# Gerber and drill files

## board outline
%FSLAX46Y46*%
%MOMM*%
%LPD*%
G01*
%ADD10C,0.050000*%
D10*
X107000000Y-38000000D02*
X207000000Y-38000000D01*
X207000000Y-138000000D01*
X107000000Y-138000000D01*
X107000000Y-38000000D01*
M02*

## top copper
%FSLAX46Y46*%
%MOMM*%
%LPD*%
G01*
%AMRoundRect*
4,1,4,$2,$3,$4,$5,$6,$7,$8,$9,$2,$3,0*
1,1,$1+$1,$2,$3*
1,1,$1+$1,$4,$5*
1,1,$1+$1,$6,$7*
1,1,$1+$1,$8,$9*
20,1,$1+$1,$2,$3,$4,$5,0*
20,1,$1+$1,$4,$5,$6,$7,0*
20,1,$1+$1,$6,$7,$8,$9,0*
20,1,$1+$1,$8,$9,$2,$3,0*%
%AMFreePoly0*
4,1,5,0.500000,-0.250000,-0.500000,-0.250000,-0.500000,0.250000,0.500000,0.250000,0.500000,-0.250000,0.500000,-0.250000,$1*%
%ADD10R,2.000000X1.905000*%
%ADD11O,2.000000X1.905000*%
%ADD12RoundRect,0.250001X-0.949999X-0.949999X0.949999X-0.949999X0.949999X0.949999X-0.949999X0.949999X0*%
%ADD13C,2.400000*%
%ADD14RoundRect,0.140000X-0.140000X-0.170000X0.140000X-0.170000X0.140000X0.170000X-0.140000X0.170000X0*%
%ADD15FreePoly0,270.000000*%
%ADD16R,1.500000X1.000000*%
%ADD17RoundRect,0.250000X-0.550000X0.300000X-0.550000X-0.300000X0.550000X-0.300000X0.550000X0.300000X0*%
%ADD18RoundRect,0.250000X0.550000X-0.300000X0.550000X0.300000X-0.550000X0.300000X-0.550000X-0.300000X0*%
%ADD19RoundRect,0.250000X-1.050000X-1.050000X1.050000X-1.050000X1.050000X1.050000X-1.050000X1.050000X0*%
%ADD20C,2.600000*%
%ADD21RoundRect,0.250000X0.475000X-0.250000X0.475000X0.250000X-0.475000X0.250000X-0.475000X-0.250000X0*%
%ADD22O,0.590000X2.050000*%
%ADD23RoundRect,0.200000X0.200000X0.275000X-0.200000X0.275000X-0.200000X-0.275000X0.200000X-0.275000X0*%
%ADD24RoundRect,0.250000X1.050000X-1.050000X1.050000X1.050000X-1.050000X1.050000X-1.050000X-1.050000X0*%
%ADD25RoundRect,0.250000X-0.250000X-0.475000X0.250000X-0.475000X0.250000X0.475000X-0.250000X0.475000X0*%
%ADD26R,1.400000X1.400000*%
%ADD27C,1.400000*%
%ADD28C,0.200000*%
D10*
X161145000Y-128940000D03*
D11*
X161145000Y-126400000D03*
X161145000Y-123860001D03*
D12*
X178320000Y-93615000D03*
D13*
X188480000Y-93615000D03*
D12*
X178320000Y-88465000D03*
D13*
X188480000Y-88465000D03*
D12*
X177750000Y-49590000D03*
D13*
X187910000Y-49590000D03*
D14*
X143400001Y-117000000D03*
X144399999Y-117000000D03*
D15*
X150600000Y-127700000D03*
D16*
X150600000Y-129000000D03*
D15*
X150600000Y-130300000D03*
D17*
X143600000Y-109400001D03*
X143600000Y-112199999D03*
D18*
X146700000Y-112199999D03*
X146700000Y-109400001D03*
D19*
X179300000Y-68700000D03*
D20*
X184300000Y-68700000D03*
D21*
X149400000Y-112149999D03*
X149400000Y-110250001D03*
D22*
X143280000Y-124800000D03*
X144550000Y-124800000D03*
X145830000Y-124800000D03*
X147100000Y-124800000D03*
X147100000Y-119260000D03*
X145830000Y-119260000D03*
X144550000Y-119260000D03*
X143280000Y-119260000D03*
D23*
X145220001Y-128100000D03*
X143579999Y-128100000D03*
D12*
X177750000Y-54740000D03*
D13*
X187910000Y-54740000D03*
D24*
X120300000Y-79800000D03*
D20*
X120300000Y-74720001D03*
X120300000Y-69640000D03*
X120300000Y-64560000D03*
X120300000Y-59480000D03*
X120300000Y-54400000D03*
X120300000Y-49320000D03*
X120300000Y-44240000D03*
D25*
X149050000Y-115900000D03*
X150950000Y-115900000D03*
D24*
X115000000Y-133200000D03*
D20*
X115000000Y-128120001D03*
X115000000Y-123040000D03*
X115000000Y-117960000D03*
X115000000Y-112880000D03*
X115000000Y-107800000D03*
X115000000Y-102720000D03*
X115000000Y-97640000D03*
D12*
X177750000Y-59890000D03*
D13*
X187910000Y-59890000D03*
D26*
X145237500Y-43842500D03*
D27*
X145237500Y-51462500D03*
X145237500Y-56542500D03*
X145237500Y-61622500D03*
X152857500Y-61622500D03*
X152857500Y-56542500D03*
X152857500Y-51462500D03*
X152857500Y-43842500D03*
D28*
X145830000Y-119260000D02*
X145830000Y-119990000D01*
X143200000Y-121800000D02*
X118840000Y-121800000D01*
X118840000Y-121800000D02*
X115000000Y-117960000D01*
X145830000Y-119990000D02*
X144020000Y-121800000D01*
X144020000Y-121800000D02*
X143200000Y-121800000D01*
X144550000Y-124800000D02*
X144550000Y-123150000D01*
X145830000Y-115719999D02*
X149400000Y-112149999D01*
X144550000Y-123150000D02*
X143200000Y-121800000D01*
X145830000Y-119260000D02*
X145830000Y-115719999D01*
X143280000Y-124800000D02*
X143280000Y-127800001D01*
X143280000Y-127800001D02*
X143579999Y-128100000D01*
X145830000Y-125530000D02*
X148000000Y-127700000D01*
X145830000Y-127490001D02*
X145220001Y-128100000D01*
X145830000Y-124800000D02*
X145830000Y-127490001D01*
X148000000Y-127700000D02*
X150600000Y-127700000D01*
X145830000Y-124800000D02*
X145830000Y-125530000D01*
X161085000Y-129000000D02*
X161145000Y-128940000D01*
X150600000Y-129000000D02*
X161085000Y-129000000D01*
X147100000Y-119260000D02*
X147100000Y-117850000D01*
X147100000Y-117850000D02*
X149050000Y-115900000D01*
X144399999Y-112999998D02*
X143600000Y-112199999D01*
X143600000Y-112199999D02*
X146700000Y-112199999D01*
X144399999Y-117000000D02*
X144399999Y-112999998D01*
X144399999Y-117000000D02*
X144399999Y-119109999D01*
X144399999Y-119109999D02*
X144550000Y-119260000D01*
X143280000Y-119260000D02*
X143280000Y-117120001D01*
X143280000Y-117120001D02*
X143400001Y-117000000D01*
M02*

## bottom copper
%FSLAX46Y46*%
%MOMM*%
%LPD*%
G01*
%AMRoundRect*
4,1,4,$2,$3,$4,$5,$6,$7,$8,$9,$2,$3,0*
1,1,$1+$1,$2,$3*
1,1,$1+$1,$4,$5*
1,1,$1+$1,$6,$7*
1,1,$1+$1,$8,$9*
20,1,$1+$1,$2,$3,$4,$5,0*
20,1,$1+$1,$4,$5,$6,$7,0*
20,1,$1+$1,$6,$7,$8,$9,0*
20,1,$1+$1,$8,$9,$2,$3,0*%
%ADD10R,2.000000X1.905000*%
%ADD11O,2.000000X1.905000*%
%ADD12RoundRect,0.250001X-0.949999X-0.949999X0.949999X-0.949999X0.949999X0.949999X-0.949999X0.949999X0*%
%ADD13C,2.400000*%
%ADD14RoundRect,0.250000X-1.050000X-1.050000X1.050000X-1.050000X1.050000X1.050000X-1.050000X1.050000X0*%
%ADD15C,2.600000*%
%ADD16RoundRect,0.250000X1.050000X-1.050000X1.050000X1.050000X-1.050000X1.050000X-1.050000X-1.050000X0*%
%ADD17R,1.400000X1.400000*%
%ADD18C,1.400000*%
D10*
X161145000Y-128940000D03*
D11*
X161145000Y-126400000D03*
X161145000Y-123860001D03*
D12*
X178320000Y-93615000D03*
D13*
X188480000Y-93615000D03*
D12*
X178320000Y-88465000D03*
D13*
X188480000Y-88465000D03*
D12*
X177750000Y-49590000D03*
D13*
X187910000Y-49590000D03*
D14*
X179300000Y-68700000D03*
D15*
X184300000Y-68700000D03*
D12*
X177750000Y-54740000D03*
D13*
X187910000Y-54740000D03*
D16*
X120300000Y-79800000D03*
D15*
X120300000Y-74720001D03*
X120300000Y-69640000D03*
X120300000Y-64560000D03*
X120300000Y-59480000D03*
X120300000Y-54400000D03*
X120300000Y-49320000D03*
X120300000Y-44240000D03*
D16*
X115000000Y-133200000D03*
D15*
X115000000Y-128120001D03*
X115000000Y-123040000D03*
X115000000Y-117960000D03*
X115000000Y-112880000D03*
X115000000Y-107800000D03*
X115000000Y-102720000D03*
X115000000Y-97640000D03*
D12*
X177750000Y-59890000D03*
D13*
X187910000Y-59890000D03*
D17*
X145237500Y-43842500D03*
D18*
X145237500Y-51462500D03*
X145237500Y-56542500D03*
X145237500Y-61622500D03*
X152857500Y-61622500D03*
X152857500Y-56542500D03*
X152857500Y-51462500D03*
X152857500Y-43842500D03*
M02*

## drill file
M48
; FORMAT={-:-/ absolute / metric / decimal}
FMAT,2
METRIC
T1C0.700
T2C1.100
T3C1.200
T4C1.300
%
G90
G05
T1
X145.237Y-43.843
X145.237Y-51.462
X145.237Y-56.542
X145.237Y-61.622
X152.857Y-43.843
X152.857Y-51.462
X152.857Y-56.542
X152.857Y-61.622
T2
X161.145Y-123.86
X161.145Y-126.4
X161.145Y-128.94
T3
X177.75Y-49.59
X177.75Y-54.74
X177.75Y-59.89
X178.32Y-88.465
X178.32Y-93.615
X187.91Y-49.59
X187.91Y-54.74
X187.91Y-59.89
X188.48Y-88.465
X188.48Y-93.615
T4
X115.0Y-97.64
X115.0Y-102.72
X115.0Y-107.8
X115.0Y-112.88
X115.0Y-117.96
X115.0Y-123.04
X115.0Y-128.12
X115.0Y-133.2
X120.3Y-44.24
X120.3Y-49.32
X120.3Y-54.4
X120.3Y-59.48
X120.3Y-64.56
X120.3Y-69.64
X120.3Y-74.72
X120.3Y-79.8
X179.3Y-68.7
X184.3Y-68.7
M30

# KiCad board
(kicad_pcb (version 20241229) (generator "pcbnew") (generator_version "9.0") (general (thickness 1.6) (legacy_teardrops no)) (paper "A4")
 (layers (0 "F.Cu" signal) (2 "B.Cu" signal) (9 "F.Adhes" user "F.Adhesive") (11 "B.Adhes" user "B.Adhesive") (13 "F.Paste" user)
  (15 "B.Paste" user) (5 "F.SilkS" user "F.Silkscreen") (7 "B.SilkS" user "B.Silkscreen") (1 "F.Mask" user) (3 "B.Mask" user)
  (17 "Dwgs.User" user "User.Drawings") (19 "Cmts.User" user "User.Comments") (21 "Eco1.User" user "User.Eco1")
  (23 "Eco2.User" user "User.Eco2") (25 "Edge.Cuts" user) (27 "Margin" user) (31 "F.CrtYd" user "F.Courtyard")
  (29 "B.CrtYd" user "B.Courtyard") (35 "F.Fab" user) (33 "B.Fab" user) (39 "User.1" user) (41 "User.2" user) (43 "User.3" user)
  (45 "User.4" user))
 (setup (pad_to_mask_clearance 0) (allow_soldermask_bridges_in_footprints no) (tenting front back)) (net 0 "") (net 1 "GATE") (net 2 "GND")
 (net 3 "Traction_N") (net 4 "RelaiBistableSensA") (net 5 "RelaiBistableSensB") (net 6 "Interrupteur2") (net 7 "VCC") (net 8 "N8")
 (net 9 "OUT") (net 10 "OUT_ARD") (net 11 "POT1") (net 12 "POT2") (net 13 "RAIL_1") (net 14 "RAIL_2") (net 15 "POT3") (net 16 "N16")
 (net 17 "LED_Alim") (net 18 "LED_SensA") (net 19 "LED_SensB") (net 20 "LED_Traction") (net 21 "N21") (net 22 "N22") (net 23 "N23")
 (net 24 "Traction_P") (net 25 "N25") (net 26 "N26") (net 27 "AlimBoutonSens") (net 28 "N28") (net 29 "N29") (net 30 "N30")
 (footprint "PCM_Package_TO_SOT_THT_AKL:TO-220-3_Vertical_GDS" (layer "F.Cu") (at 161.145 128.94 90)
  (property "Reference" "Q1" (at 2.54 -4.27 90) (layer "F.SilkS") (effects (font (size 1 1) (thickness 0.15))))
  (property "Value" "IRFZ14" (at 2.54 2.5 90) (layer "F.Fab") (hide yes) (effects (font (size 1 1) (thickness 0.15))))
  (pad "1" thru_hole rect (at 0 0 90) (size 1.905 2) (drill 1.1) (layers "*.Cu" "*.Mask") (remove_unused_layers no) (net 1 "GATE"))
  (pad "2" thru_hole oval (at 2.54 0 90) (size 1.905 2) (drill 1.1) (layers "*.Cu" "*.Mask") (remove_unused_layers no) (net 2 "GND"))
  (pad "3" thru_hole oval (at 5.079999 0 90) (size 1.905 2) (drill 1.1) (layers "*.Cu" "*.Mask") (remove_unused_layers no)
   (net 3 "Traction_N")))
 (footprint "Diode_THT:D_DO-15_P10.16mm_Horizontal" (layer "F.Cu") (at 178.32 93.615)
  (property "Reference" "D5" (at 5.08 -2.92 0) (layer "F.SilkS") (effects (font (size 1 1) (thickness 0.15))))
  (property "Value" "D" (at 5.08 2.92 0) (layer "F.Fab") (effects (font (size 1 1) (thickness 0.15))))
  (pad "1" thru_hole roundrect (at 0 0) (size 2.4 2.4) (drill 1.2) (layers "*.Cu" "*.Mask") (remove_unused_layers no)
   (roundrect_rratio 0.104167) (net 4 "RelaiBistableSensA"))
  (pad "2" thru_hole circle (at 10.16 0) (size 2.4 2.4) (drill 1.2) (layers "*.Cu" "*.Mask") (remove_unused_layers no) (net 2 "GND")))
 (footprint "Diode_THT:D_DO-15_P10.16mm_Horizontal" (layer "F.Cu") (at 178.32 88.465)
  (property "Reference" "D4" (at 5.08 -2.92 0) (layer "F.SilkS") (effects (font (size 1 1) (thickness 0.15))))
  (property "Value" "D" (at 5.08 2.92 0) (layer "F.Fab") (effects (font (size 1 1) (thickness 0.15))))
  (pad "1" thru_hole roundrect (at 0 0) (size 2.4 2.4) (drill 1.2) (layers "*.Cu" "*.Mask") (remove_unused_layers no)
   (roundrect_rratio 0.104167) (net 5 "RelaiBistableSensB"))
  (pad "2" thru_hole circle (at 10.16 0) (size 2.4 2.4) (drill 1.2) (layers "*.Cu" "*.Mask") (remove_unused_layers no) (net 2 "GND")))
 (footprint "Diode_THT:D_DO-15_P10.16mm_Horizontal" (layer "F.Cu") (at 177.75 49.59)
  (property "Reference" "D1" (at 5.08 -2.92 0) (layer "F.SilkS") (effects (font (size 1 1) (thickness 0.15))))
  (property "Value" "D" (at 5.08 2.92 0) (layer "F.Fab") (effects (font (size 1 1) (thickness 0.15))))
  (pad "1" thru_hole roundrect (at 0 0) (size 2.4 2.4) (drill 1.2) (layers "*.Cu" "*.Mask") (remove_unused_layers no)
   (roundrect_rratio 0.104167) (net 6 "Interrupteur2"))
  (pad "2" thru_hole circle (at 10.16 0) (size 2.4 2.4) (drill 1.2) (layers "*.Cu" "*.Mask") (remove_unused_layers no) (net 2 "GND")))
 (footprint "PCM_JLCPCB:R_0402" (layer "F.Cu") (at 143.9 117)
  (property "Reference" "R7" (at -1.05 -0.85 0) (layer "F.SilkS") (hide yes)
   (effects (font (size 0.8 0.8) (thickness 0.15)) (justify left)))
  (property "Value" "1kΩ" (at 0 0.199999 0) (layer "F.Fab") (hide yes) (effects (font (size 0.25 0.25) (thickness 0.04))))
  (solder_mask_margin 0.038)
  (pad "1" smd roundrect (at -0.499999 0) (size 0.56 0.62) (layers "F.Cu" "F.Mask" "F.Paste") (roundrect_rratio 0.25) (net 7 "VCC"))
  (pad "2" smd roundrect (at 0.499999 0) (size 0.56 0.62) (layers "F.Cu" "F.Mask" "F.Paste") (roundrect_rratio 0.25) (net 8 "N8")))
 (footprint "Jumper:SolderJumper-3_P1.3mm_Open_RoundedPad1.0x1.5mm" (layer "F.Cu") (at 150.6 129 -90)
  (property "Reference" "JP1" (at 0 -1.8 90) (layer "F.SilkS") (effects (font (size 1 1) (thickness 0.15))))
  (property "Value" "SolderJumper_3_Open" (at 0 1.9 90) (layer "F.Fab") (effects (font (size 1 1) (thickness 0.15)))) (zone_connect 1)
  (pad "1" smd custom (at -1.3 0 270) (size 1 0.5) (layers "F.Cu" "F.Mask") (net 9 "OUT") (zone_connect 2) (thermal_bridge_angle 45)
   (options (clearance outline) (anchor rect)) (primitives))
  (pad "2" smd rect (at 0 0 270) (size 1 1.5) (layers "F.Cu" "F.Mask") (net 1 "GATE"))
  (pad "3" smd custom (at 1.3 0 270) (size 1 0.5) (layers "F.Cu" "F.Mask") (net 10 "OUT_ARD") (zone_connect 2) (thermal_bridge_angle 45)
   (options (clearance outline) (anchor rect)) (primitives)))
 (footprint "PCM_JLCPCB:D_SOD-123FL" (layer "F.Cu") (at 143.6 110.8 -90)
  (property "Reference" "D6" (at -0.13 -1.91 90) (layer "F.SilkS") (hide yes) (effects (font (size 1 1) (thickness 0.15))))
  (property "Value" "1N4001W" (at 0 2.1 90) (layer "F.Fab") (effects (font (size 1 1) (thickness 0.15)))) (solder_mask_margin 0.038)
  (pad "1" smd roundrect (at -1.399999 0 270) (size 1.1 1.6) (layers "F.Cu" "F.Mask" "F.Paste") (roundrect_rratio 0.2272727273)
   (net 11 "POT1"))
  (pad "2" smd roundrect (at 1.399999 0 270) (size 1.1 1.6) (layers "F.Cu" "F.Mask" "F.Paste") (roundrect_rratio 0.2272727273) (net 8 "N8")))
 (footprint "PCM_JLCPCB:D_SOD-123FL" (layer "F.Cu") (at 146.7 110.8 90)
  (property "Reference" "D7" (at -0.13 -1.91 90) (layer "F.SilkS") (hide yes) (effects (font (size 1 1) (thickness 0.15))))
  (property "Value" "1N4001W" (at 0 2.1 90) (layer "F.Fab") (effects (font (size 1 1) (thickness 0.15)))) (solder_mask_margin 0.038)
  (pad "1" smd roundrect (at -1.399999 0 90) (size 1.1 1.6) (layers "F.Cu" "F.Mask" "F.Paste") (roundrect_rratio 0.2272727273) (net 8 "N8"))
  (pad "2" smd roundrect (at 1.399999 0 90) (size 1.1 1.6) (layers "F.Cu" "F.Mask" "F.Paste") (roundrect_rratio 0.2272727273)
   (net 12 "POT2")))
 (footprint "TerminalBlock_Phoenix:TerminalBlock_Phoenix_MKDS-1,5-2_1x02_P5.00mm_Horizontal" (layer "F.Cu") (at 179.3 68.7)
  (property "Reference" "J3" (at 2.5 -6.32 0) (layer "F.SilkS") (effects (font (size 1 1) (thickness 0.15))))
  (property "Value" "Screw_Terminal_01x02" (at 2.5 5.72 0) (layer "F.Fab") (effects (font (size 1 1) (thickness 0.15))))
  (pad "1" thru_hole roundrect (at 0 0) (size 2.6 2.6) (drill 1.3) (layers "*.Cu" "*.Mask") (remove_unused_layers no)
   (roundrect_rratio 0.096154) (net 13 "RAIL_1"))
  (pad "2" thru_hole circle (at 5 0) (size 2.6 2.6) (drill 1.3) (layers "*.Cu" "*.Mask") (remove_unused_layers no) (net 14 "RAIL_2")))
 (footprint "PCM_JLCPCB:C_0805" (layer "F.Cu") (at 149.4 111.2 90)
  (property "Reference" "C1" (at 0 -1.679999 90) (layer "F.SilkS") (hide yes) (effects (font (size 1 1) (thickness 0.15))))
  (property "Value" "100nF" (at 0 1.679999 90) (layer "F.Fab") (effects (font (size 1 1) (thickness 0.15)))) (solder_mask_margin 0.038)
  (pad "1" smd roundrect (at -0.949999 0 90) (size 1 1.45) (layers "F.Cu" "F.Mask" "F.Paste") (roundrect_rratio 0.25) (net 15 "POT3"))
  (pad "2" smd roundrect (at 0.949999 0 90) (size 1 1.45) (layers "F.Cu" "F.Mask" "F.Paste") (roundrect_rratio 0.25) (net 2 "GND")))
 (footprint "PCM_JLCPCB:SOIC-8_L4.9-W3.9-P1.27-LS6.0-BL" (layer "F.Cu") (at 145.19 122.03)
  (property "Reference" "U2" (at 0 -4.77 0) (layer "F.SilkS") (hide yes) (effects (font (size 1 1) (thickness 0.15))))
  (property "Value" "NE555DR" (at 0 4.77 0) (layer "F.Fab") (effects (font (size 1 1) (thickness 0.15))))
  (pad "1" smd oval (at -1.91 2.77) (size 0.59 2.05) (layers "F.Cu" "F.Mask" "F.Paste") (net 2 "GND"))
  (pad "2" smd oval (at -0.64 2.77) (size 0.59 2.05) (layers "F.Cu" "F.Mask" "F.Paste") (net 15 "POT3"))
  (pad "3" smd oval (at 0.64 2.77) (size 0.59 2.05) (layers "F.Cu" "F.Mask" "F.Paste") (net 9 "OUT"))
  (pad "4" smd oval (at 1.91 2.77) (size 0.59 2.05) (layers "F.Cu" "F.Mask" "F.Paste") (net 7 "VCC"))
  (pad "5" smd oval (at 1.91 -2.77) (size 0.59 2.05) (layers "F.Cu" "F.Mask" "F.Paste") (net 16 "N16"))
  (pad "6" smd oval (at 0.64 -2.77) (size 0.59 2.05) (layers "F.Cu" "F.Mask" "F.Paste") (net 15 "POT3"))
  (pad "7" smd oval (at -0.64 -2.77) (size 0.59 2.05) (layers "F.Cu" "F.Mask" "F.Paste") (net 8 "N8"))
  (pad "8" smd oval (at -1.91 -2.77) (size 0.59 2.05) (layers "F.Cu" "F.Mask" "F.Paste") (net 7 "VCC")))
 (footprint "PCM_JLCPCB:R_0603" (layer "F.Cu") (at 144.4 128.1 180)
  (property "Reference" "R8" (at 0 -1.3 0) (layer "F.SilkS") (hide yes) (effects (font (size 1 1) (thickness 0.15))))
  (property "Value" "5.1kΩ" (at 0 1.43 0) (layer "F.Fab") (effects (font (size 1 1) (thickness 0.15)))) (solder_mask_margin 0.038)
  (pad "1" smd roundrect (at -0.820001 0 180) (size 0.8 0.95) (layers "F.Cu" "F.Mask" "F.Paste") (roundrect_rratio 0.25) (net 9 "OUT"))
  (pad "2" smd roundrect (at 0.820001 0 180) (size 0.8 0.95) (layers "F.Cu" "F.Mask" "F.Paste") (roundrect_rratio 0.25) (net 2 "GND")))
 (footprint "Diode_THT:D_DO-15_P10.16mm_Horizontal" (layer "F.Cu") (at 177.75 54.74)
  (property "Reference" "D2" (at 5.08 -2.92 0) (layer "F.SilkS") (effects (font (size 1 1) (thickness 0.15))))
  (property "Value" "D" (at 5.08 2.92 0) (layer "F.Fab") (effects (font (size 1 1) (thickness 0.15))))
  (pad "1" thru_hole roundrect (at 0 0) (size 2.4 2.4) (drill 1.2) (layers "*.Cu" "*.Mask") (remove_unused_layers no)
   (roundrect_rratio 0.104167) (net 5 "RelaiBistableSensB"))
  (pad "2" thru_hole circle (at 10.16 0) (size 2.4 2.4) (drill 1.2) (layers "*.Cu" "*.Mask") (remove_unused_layers no) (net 2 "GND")))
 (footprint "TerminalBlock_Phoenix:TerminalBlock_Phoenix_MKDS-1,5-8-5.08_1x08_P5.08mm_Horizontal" (layer "F.Cu") (at 120.3 79.8 90)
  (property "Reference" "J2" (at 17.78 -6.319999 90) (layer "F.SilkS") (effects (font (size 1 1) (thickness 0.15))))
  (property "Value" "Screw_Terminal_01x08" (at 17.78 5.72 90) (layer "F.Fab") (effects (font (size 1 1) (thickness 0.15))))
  (pad "1" thru_hole roundrect (at 0 0 90) (size 2.6 2.6) (drill 1.3) (layers "*.Cu" "*.Mask") (remove_unused_layers no)
   (roundrect_rratio 0.096154) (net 2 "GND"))
  (pad "2" thru_hole circle (at 5.079999 0 90) (size 2.6 2.6) (drill 1.3) (layers "*.Cu" "*.Mask") (remove_unused_layers no)
   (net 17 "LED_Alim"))
  (pad "3" thru_hole circle (at 10.16 0 90) (size 2.6 2.6) (drill 1.3) (layers "*.Cu" "*.Mask") (remove_unused_layers no)
   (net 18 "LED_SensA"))
  (pad "4" thru_hole circle (at 15.24 0 90) (size 2.6 2.6) (drill 1.3) (layers "*.Cu" "*.Mask") (remove_unused_layers no)
   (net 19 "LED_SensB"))
  (pad "5" thru_hole circle (at 20.32 0 90) (size 2.6 2.6) (drill 1.3) (layers "*.Cu" "*.Mask") (remove_unused_layers no)
   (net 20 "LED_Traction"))
  (pad "6" thru_hole circle (at 25.4 0 90) (size 2.6 2.6) (drill 1.3) (layers "*.Cu" "*.Mask") (remove_unused_layers no) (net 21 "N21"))
  (pad "7" thru_hole circle (at 30.48 0 90) (size 2.6 2.6) (drill 1.3) (layers "*.Cu" "*.Mask") (remove_unused_layers no) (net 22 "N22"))
  (pad "8" thru_hole circle (at 35.56 0 90) (size 2.6 2.6) (drill 1.3) (layers "*.Cu" "*.Mask") (remove_unused_layers no) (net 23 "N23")))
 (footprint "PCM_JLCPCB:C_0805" (layer "F.Cu") (at 150 115.9)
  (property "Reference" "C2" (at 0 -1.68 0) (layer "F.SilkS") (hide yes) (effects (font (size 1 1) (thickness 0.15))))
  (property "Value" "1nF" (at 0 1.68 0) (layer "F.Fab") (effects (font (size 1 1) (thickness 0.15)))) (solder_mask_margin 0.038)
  (pad "1" smd roundrect (at -0.95 0) (size 1 1.45) (layers "F.Cu" "F.Mask" "F.Paste") (roundrect_rratio 0.25) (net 16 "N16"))
  (pad "2" smd roundrect (at 0.95 0) (size 1 1.45) (layers "F.Cu" "F.Mask" "F.Paste") (roundrect_rratio 0.25) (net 2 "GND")))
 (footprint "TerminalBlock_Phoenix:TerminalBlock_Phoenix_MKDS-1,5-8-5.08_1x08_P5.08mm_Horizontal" (layer "F.Cu") (at 115 133.2 90)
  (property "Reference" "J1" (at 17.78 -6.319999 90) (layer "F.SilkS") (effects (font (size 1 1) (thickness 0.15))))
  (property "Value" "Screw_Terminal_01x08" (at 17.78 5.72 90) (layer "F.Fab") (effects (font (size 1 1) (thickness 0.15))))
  (pad "1" thru_hole roundrect (at 0 0 90) (size 2.6 2.6) (drill 1.3) (layers "*.Cu" "*.Mask") (remove_unused_layers no)
   (roundrect_rratio 0.096154) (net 2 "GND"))
  (pad "2" thru_hole circle (at 5.079999 0 90) (size 2.6 2.6) (drill 1.3) (layers "*.Cu" "*.Mask") (remove_unused_layers no) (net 11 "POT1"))
  (pad "3" thru_hole circle (at 10.16 0 90) (size 2.6 2.6) (drill 1.3) (layers "*.Cu" "*.Mask") (remove_unused_layers no) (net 12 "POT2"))
  (pad "4" thru_hole circle (at 15.24 0 90) (size 2.6 2.6) (drill 1.3) (layers "*.Cu" "*.Mask") (remove_unused_layers no) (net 15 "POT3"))
  (pad "5" thru_hole circle (at 20.32 0 90) (size 2.6 2.6) (drill 1.3) (layers "*.Cu" "*.Mask") (remove_unused_layers no) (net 10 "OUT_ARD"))
  (pad "6" thru_hole circle (at 25.4 0 90) (size 2.6 2.6) (drill 1.3) (layers "*.Cu" "*.Mask") (remove_unused_layers no)
   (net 3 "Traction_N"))
  (pad "7" thru_hole circle (at 30.48 0 90) (size 2.6 2.6) (drill 1.3) (layers "*.Cu" "*.Mask") (remove_unused_layers no)
   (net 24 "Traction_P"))
  (pad "8" thru_hole circle (at 35.56 0 90) (size 2.6 2.6) (drill 1.3) (layers "*.Cu" "*.Mask") (remove_unused_layers no) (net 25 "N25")))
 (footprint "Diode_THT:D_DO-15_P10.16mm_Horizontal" (layer "F.Cu") (at 177.75 59.89)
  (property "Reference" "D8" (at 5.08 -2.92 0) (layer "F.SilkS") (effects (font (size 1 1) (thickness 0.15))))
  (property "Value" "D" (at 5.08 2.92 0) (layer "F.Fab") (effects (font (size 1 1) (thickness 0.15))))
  (pad "1" thru_hole roundrect (at 0 0) (size 2.4 2.4) (drill 1.2) (layers "*.Cu" "*.Mask") (remove_unused_layers no)
   (roundrect_rratio 0.104167) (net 4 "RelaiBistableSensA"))
  (pad "2" thru_hole circle (at 10.16 0) (size 2.4 2.4) (drill 1.2) (layers "*.Cu" "*.Mask") (remove_unused_layers no) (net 2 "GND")))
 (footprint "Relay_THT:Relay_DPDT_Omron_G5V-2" (layer "F.Cu") (at 145.2375 43.8425)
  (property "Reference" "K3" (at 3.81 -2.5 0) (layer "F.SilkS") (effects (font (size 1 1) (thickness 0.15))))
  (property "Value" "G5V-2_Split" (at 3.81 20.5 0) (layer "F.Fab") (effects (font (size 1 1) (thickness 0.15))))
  (pad "1" thru_hole rect (at 0 0) (size 1.4 1.4) (drill 0.7) (layers "*.Cu" "*.Mask") (remove_unused_layers no) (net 2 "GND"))
  (pad "4" thru_hole circle (at 0 7.62) (size 1.4 1.4) (drill 0.7) (layers "*.Cu" "*.Mask") (remove_unused_layers no) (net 7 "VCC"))
  (pad "6" thru_hole circle (at 0 12.7) (size 1.4 1.4) (drill 0.7) (layers "*.Cu" "*.Mask") (remove_unused_layers no) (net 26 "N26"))
  (pad "8" thru_hole circle (at 0 17.78) (size 1.4 1.4) (drill 0.7) (layers "*.Cu" "*.Mask") (remove_unused_layers no)
   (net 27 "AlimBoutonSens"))
  (pad "9" thru_hole circle (at 7.62 17.78) (size 1.4 1.4) (drill 0.7) (layers "*.Cu" "*.Mask") (remove_unused_layers no) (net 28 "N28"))
  (pad "11" thru_hole circle (at 7.62 12.7) (size 1.4 1.4) (drill 0.7) (layers "*.Cu" "*.Mask") (remove_unused_layers no) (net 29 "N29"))
  (pad "13" thru_hole circle (at 7.62 7.62) (size 1.4 1.4) (drill 0.7) (layers "*.Cu" "*.Mask") (remove_unused_layers no) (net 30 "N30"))
  (pad "16" thru_hole circle (at 7.62 0) (size 1.4 1.4) (drill 0.7) (layers "*.Cu" "*.Mask") (remove_unused_layers no)
   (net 6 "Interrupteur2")))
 (gr_rect (start 107 38) (end 207 138) (stroke (width 0.05) (type default)) (fill no) (layer "Edge.Cuts"))
 (segment (start 145.83 119.26) (end 145.83 119.99) (width 0.2) (layer "F.Cu") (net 15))
 (segment (start 143.2 121.8) (end 118.84 121.8) (width 0.2) (layer "F.Cu") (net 15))
 (segment (start 118.84 121.8) (end 115 117.96) (width 0.2) (layer "F.Cu") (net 15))
 (segment (start 145.83 119.99) (end 144.02 121.8) (width 0.2) (layer "F.Cu") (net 15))
 (segment (start 144.02 121.8) (end 143.2 121.8) (width 0.2) (layer "F.Cu") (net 15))
 (segment (start 144.55 124.8) (end 144.55 123.15) (width 0.2) (layer "F.Cu") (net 15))
 (segment (start 145.83 115.719999) (end 149.4 112.149999) (width 0.2) (layer "F.Cu") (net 15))
 (segment (start 144.55 123.15) (end 143.2 121.8) (width 0.2) (layer "F.Cu") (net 15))
 (segment (start 145.83 119.26) (end 145.83 115.719999) (width 0.2) (layer "F.Cu") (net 15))
 (segment (start 143.28 124.8) (end 143.28 127.800001) (width 0.2) (layer "F.Cu") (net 2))
 (segment (start 143.28 127.800001) (end 143.579999 128.1) (width 0.2) (layer "F.Cu") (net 2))
 (segment (start 145.83 125.53) (end 148 127.7) (width 0.2) (layer "F.Cu") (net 9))
 (segment (start 145.83 127.490001) (end 145.220001 128.1) (width 0.2) (layer "F.Cu") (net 9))
 (segment (start 145.83 124.8) (end 145.83 127.490001) (width 0.2) (layer "F.Cu") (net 9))
 (segment (start 148 127.7) (end 150.6 127.7) (width 0.2) (layer "F.Cu") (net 9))
 (segment (start 145.83 124.8) (end 145.83 125.53) (width 0.2) (layer "F.Cu") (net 9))
 (segment (start 161.085 129) (end 161.145 128.94) (width 0.2) (layer "F.Cu") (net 1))
 (segment (start 150.6 129) (end 161.085 129) (width 0.2) (layer "F.Cu") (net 1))
 (segment (start 147.1 119.26) (end 147.1 117.85) (width 0.2) (layer "F.Cu") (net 16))
 (segment (start 147.1 117.85) (end 149.05 115.9) (width 0.2) (layer "F.Cu") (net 16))
 (segment (start 144.399999 112.999998) (end 143.6 112.199999) (width 0.2) (layer "F.Cu") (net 8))
 (segment (start 143.6 112.199999) (end 146.7 112.199999) (width 0.2) (layer "F.Cu") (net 8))
 (segment (start 144.399999 117) (end 144.399999 112.999998) (width 0.2) (layer "F.Cu") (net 8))
 (segment (start 144.399999 117) (end 144.399999 119.109999) (width 0.2) (layer "F.Cu") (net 8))
 (segment (start 144.399999 119.109999) (end 144.55 119.26) (width 0.2) (layer "F.Cu") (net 8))
 (segment (start 143.28 119.26) (end 143.28 117.120001) (width 0.2) (layer "F.Cu") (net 7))
 (segment (start 143.28 117.120001) (end 143.400001 117) (width 0.2) (layer "F.Cu") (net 7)))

